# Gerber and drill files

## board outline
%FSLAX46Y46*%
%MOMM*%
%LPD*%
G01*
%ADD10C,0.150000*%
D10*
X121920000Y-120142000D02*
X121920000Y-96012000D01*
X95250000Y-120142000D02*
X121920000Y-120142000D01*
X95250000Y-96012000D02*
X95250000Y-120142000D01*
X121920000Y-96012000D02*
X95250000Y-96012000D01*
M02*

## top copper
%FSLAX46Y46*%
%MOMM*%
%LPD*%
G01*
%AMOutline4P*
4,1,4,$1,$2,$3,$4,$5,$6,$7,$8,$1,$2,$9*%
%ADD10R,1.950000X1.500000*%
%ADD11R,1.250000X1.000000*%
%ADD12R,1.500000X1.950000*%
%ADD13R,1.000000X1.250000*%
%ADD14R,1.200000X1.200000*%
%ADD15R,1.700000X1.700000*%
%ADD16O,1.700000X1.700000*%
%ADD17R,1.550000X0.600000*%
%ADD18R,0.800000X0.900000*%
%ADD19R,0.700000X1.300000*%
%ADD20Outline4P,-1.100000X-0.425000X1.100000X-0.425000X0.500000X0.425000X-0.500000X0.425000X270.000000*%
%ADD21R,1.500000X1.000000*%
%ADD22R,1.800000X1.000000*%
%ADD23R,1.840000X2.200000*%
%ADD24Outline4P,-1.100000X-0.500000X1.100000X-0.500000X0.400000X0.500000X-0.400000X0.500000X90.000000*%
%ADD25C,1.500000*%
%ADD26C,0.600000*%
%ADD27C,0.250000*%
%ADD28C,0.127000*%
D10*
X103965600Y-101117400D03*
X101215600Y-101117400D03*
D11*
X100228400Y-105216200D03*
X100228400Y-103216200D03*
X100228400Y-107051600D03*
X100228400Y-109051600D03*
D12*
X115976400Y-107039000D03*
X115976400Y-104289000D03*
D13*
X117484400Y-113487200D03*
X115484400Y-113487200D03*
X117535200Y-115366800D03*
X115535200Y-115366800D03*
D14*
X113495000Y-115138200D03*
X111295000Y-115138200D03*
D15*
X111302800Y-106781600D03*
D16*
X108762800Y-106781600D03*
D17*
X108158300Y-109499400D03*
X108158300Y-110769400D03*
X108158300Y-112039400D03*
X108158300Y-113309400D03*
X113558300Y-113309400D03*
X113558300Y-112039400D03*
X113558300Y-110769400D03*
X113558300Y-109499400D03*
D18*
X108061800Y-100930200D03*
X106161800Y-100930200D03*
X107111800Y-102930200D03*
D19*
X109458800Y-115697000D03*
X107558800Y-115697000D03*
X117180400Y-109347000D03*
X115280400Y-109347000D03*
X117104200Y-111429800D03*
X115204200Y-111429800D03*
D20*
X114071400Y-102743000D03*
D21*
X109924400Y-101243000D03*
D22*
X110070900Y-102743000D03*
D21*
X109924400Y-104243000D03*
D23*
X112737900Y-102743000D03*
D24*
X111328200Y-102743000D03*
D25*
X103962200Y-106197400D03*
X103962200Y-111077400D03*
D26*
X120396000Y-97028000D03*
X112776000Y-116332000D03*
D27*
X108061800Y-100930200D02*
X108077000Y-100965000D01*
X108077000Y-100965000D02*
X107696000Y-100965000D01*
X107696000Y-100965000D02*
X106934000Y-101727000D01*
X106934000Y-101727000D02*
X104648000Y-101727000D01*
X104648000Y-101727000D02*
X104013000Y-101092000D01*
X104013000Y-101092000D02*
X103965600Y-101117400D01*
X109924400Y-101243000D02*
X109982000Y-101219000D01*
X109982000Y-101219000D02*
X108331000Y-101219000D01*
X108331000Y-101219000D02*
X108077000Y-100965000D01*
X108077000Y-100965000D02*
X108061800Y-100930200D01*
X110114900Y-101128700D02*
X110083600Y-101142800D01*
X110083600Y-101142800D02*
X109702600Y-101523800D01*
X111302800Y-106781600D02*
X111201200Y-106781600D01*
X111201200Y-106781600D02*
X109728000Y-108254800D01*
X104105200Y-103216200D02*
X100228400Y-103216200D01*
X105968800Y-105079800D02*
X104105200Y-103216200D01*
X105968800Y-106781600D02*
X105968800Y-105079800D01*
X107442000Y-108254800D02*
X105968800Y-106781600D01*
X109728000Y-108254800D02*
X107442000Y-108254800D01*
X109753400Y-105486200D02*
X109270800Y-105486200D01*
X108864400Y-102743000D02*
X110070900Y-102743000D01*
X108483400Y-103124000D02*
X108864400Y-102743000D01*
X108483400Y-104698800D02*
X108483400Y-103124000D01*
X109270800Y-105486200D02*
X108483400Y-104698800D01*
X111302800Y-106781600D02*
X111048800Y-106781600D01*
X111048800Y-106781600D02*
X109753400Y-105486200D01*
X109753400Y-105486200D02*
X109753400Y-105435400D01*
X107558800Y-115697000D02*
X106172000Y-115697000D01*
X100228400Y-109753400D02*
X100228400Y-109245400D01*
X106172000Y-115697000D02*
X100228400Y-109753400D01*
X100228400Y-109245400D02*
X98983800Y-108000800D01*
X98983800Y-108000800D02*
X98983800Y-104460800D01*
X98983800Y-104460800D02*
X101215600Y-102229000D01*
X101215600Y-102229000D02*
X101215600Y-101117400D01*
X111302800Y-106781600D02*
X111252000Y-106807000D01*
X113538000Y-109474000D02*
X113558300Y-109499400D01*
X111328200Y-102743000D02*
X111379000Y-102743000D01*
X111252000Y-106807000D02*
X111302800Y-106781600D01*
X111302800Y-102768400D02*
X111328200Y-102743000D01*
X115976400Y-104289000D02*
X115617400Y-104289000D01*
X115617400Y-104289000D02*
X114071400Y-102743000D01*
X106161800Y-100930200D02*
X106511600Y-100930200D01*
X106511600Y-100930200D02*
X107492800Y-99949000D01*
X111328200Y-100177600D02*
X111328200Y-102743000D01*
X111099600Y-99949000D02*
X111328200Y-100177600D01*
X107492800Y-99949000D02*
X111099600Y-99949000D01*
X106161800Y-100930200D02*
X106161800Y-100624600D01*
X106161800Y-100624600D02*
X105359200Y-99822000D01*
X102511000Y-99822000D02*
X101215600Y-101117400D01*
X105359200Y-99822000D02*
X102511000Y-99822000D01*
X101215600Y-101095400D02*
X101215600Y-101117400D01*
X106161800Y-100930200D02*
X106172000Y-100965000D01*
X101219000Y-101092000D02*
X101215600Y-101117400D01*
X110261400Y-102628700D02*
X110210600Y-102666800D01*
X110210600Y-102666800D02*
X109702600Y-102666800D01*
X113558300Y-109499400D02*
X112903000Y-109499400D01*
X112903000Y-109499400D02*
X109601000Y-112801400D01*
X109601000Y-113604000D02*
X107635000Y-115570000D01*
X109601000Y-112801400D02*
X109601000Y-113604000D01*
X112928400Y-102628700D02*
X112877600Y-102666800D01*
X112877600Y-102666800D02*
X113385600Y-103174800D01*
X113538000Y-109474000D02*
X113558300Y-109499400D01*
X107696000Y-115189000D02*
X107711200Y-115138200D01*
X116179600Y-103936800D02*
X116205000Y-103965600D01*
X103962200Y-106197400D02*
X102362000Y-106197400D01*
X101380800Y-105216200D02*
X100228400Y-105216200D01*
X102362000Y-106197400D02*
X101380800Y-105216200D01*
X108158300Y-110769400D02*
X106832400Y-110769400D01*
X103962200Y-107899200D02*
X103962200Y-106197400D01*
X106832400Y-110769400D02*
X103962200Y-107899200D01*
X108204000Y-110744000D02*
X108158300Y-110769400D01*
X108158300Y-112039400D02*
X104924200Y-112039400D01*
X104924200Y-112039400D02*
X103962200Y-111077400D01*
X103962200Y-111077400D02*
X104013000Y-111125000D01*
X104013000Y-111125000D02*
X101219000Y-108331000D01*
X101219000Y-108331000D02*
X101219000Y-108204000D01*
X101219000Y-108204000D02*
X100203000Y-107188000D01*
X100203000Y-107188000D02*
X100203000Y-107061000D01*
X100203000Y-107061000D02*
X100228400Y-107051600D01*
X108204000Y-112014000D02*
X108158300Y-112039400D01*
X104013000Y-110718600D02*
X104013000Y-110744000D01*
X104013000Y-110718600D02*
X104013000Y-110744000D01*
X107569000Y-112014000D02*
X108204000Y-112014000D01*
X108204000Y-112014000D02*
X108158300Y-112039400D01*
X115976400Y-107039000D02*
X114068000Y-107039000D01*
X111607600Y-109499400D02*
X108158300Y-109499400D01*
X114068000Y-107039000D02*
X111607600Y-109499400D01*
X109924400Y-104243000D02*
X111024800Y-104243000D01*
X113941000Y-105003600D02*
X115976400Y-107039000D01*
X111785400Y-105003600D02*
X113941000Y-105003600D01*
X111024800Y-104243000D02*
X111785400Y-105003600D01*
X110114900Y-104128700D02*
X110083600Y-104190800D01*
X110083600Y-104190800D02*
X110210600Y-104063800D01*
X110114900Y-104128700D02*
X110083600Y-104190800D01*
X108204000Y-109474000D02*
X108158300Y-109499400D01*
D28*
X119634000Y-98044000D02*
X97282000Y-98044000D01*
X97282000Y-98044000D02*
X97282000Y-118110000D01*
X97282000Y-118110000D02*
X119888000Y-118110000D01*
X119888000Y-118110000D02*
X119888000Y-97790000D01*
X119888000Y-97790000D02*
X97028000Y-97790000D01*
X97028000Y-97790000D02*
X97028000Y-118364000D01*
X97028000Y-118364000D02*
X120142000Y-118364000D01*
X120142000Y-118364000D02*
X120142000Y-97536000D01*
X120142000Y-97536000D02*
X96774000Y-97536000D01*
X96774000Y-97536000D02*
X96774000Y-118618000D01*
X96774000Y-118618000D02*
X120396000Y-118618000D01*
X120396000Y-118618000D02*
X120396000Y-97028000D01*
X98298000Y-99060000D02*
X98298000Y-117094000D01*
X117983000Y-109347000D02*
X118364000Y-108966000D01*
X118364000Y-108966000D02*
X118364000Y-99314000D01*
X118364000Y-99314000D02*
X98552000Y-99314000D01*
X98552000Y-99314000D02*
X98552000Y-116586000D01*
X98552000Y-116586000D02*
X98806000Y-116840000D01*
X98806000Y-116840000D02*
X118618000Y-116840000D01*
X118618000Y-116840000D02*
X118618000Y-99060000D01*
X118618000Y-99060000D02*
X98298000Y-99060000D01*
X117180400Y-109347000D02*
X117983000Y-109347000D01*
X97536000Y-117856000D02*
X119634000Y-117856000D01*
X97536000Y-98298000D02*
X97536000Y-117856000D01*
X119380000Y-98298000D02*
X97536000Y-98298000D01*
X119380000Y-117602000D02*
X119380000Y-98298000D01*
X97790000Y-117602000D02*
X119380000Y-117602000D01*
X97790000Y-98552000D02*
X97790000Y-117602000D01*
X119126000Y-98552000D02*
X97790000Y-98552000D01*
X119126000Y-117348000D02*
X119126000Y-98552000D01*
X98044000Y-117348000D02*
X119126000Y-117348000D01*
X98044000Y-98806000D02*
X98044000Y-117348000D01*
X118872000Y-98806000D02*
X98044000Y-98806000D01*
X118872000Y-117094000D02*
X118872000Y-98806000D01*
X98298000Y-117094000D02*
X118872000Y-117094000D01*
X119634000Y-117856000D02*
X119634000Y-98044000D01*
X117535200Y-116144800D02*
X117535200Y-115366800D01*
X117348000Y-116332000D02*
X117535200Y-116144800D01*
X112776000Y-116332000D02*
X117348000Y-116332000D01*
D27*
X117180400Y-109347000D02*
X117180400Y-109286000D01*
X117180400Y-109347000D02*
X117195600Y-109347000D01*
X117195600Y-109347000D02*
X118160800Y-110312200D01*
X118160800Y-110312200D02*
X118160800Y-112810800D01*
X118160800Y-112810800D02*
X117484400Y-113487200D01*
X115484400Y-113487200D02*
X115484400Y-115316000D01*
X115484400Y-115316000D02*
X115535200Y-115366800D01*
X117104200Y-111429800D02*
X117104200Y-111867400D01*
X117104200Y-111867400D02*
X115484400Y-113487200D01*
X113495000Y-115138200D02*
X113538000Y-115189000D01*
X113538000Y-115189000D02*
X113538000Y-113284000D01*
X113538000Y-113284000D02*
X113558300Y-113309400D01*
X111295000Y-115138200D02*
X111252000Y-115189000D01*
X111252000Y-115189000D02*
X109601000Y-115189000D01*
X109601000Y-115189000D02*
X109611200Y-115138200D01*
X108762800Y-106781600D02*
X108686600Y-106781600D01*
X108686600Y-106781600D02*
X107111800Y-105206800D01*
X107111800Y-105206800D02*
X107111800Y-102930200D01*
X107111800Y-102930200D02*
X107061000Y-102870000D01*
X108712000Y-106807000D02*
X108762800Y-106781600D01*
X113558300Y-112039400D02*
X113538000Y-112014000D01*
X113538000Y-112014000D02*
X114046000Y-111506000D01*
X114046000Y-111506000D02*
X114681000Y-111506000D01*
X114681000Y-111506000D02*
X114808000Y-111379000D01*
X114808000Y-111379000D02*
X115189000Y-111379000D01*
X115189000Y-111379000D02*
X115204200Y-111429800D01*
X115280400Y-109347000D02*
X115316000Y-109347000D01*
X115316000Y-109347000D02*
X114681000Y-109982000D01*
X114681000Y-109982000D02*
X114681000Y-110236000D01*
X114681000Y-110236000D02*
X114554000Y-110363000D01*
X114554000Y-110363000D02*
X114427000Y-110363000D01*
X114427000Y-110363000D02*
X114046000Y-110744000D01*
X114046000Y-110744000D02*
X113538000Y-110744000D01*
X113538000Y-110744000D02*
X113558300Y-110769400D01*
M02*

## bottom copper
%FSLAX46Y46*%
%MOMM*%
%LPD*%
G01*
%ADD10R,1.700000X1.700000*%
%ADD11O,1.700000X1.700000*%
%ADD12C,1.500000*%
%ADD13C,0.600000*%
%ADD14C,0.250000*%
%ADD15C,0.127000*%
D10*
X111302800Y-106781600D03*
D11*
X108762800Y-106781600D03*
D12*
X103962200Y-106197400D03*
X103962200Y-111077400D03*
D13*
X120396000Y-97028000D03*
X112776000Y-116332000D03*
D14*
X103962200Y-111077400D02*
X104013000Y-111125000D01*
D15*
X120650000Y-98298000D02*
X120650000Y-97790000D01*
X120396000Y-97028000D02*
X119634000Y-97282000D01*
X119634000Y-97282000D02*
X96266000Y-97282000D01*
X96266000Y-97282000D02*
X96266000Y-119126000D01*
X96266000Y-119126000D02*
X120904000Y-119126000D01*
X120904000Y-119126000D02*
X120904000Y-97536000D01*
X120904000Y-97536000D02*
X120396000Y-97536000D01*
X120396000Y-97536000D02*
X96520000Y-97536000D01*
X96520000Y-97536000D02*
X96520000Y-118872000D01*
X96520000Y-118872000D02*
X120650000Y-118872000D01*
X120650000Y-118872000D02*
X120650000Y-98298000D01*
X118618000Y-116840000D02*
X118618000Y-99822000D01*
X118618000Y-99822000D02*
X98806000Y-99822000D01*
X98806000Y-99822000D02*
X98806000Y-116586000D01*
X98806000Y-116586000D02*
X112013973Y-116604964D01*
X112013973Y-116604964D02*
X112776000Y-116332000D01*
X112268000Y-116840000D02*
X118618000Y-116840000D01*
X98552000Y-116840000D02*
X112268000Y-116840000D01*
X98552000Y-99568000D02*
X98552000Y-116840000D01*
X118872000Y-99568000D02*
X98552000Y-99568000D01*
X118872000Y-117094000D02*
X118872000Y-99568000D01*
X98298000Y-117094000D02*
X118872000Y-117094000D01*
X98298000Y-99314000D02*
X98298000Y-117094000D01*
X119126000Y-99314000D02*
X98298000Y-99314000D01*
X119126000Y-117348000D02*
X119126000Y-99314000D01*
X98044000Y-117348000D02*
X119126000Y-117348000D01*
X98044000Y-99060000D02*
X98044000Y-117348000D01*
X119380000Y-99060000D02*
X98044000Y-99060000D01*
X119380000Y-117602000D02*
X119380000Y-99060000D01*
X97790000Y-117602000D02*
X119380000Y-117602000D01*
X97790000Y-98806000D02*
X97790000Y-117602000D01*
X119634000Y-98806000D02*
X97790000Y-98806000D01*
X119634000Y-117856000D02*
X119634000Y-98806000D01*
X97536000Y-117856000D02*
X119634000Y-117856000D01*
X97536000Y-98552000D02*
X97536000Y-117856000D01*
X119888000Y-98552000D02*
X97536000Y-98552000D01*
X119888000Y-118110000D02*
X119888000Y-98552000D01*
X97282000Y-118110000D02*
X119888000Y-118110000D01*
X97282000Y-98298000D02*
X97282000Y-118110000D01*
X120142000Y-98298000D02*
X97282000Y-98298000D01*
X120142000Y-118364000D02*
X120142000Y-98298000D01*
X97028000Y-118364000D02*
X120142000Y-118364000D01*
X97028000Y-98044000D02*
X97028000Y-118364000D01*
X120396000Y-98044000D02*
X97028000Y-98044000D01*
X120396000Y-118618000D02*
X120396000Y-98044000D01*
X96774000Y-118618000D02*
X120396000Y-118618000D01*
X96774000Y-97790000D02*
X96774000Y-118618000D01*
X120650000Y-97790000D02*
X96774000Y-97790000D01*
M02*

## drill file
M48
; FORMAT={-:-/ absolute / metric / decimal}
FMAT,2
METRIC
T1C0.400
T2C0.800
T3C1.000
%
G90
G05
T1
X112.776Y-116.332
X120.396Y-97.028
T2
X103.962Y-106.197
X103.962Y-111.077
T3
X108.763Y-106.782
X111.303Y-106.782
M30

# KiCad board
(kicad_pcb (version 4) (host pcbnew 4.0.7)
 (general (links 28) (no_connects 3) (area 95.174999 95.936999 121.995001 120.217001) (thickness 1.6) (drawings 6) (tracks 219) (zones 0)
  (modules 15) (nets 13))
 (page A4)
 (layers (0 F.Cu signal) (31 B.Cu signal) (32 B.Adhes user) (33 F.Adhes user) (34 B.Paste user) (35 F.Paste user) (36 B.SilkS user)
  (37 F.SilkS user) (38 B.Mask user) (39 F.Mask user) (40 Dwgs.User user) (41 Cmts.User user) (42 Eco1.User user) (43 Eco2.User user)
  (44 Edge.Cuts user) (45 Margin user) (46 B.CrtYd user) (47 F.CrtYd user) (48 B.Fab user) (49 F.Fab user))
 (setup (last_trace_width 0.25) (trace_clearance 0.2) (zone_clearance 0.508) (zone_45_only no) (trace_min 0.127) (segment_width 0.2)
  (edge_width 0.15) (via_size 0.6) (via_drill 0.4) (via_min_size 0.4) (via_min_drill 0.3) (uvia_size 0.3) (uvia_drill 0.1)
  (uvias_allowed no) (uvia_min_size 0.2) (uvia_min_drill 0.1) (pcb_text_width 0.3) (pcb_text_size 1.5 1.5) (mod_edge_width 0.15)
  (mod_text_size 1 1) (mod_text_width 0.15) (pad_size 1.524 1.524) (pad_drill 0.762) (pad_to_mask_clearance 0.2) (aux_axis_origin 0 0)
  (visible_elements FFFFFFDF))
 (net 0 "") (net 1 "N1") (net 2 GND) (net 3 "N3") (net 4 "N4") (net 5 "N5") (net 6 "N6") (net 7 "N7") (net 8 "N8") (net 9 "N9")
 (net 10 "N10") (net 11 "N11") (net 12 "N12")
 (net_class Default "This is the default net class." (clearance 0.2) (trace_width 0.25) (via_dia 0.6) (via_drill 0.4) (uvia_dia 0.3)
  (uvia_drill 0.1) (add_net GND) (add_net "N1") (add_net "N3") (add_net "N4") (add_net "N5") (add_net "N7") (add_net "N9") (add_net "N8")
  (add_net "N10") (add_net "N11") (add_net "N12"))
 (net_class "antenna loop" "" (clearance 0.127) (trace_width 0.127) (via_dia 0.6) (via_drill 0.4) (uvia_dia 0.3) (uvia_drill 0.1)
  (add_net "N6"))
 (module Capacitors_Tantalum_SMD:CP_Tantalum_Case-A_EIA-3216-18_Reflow (layer F.Cu) (at 102.5906 101.1174 180)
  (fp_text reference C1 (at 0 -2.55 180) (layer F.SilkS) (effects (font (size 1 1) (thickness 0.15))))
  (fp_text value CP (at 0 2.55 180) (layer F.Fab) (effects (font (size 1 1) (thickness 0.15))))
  (pad 1 smd rect (at -1.375 0 180) (size 1.95 1.5) (layers F.Cu F.Paste F.Mask) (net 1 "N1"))
  (pad 2 smd rect (at 1.375 0 180) (size 1.95 1.5) (layers F.Cu F.Paste F.Mask) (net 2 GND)))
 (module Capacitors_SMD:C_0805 (layer F.Cu) (at 100.2284 104.2162 90)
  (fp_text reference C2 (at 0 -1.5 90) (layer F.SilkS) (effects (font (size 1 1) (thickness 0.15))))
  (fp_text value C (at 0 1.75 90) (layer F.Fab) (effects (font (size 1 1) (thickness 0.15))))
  (pad 1 smd rect (at -1 0 90) (size 1 1.25) (layers F.Cu F.Paste F.Mask) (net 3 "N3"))
  (pad 2 smd rect (at 1 0 90) (size 1 1.25) (layers F.Cu F.Paste F.Mask) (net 2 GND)))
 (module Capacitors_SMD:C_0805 (layer F.Cu) (at 100.2284 108.0516 270)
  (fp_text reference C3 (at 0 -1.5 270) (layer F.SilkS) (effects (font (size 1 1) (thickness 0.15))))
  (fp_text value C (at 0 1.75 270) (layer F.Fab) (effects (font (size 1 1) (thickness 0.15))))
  (pad 1 smd rect (at -1 0 270) (size 1 1.25) (layers F.Cu F.Paste F.Mask) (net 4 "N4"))
  (pad 2 smd rect (at 1 0 270) (size 1 1.25) (layers F.Cu F.Paste F.Mask) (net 2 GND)))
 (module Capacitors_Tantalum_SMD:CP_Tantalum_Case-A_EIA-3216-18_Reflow (layer F.Cu) (at 115.9764 105.664 90)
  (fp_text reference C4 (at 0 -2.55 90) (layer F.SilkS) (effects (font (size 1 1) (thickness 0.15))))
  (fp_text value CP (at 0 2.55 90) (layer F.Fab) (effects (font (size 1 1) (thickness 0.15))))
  (pad 1 smd rect (at -1.375 0 90) (size 1.95 1.5) (layers F.Cu F.Paste F.Mask) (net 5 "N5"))
  (pad 2 smd rect (at 1.375 0 90) (size 1.95 1.5) (layers F.Cu F.Paste F.Mask) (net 2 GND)))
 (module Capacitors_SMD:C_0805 (layer F.Cu) (at 116.4844 113.4872 180)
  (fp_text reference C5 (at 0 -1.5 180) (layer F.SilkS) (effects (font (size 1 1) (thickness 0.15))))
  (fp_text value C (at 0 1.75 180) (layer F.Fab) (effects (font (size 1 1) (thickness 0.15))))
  (pad 1 smd rect (at -1 0 180) (size 1 1.25) (layers F.Cu F.Paste F.Mask) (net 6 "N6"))
  (pad 2 smd rect (at 1 0 180) (size 1 1.25) (layers F.Cu F.Paste F.Mask) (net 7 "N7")))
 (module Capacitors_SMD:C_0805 (layer F.Cu) (at 116.5352 115.3668 180)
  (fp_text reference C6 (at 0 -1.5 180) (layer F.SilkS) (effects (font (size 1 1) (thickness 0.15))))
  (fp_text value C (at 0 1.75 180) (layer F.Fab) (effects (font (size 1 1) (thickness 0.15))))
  (pad 1 smd rect (at -1 0 180) (size 1 1.25) (layers F.Cu F.Paste F.Mask) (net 6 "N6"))
  (pad 2 smd rect (at 1 0 180) (size 1 1.25) (layers F.Cu F.Paste F.Mask) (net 7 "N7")))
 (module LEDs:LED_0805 (layer F.Cu) (at 112.395 115.1382)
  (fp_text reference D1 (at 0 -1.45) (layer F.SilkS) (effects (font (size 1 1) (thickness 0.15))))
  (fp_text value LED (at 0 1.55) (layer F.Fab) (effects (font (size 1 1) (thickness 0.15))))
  (pad 2 smd rect (at 1.1 0 180) (size 1.2 1.2) (layers F.Cu F.Paste F.Mask) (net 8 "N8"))
  (pad 1 smd rect (at -1.1 0 180) (size 1.2 1.2) (layers F.Cu F.Paste F.Mask) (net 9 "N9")))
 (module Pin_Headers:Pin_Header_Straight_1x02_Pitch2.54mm (layer F.Cu) (at 111.3028 106.7816 270)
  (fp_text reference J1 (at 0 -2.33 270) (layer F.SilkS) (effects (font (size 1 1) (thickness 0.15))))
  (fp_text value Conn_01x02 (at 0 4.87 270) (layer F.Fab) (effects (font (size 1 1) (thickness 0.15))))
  (pad 1 thru_hole rect (at 0 0 270) (size 1.7 1.7) (drill 1) (layers *.Cu *.Mask) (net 2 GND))
  (pad 2 thru_hole oval (at 0 2.54 270) (size 1.7 1.7) (drill 1) (layers *.Cu *.Mask) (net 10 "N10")))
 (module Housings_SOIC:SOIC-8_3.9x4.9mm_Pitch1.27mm (layer F.Cu) (at 110.8583 111.4044)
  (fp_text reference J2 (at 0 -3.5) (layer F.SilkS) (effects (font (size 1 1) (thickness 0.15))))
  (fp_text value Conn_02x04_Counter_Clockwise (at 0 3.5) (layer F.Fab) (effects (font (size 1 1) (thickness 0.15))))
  (pad 1 smd rect (at -2.7 -1.905) (size 1.55 0.6) (layers F.Cu F.Paste F.Mask) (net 5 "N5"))
  (pad 2 smd rect (at -2.7 -0.635) (size 1.55 0.6) (layers F.Cu F.Paste F.Mask) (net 3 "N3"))
  (pad 3 smd rect (at -2.7 0.635) (size 1.55 0.6) (layers F.Cu F.Paste F.Mask) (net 4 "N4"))
  (pad 4 smd rect (at -2.7 1.905) (size 1.55 0.6) (layers F.Cu F.Paste F.Mask))
  (pad 5 smd rect (at 2.7 1.905) (size 1.55 0.6) (layers F.Cu F.Paste F.Mask) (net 8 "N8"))
  (pad 6 smd rect (at 2.7 0.635) (size 1.55 0.6) (layers F.Cu F.Paste F.Mask) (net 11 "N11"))
  (pad 7 smd rect (at 2.7 -0.635) (size 1.55 0.6) (layers F.Cu F.Paste F.Mask) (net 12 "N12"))
  (pad 8 smd rect (at 2.7 -1.905) (size 1.55 0.6) (layers F.Cu F.Paste F.Mask) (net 2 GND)))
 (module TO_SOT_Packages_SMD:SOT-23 (layer F.Cu) (at 107.1118 101.9302 270)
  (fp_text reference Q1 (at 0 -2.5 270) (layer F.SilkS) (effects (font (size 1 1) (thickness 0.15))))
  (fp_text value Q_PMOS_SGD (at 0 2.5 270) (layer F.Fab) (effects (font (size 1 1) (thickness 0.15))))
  (pad 1 smd rect (at -1 -0.95 270) (size 0.9 0.8) (layers F.Cu F.Paste F.Mask) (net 1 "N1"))
  (pad 2 smd rect (at -1 0.95 270) (size 0.9 0.8) (layers F.Cu F.Paste F.Mask) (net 2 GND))
  (pad 3 smd rect (at 1 0 270) (size 0.9 0.8) (layers F.Cu F.Paste F.Mask) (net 10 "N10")))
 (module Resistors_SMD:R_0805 (layer F.Cu) (at 108.5088 115.697 180)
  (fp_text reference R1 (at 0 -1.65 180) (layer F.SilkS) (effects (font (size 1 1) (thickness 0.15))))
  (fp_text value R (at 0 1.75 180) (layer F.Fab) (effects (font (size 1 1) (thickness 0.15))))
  (pad 1 smd rect (at -0.95 0 180) (size 0.7 1.3) (layers F.Cu F.Paste F.Mask) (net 9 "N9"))
  (pad 2 smd rect (at 0.95 0 180) (size 0.7 1.3) (layers F.Cu F.Paste F.Mask) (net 2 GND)))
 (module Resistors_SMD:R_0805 (layer F.Cu) (at 116.2304 109.347 180)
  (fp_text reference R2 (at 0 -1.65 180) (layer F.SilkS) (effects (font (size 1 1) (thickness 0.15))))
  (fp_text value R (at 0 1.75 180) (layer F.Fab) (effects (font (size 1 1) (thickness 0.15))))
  (pad 1 smd rect (at -0.95 0 180) (size 0.7 1.3) (layers F.Cu F.Paste F.Mask) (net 6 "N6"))
  (pad 2 smd rect (at 0.95 0 180) (size 0.7 1.3) (layers F.Cu F.Paste F.Mask) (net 12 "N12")))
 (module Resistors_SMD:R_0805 (layer F.Cu) (at 116.1542 111.4298 180)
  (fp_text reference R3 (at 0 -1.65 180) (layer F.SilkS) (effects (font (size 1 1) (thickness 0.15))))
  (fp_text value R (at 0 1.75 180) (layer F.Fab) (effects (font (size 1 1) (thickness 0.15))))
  (pad 1 smd rect (at -0.95 0 180) (size 0.7 1.3) (layers F.Cu F.Paste F.Mask) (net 7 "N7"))
  (pad 2 smd rect (at 0.95 0 180) (size 0.7 1.3) (layers F.Cu F.Paste F.Mask) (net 11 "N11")))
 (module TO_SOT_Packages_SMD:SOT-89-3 (layer F.Cu) (at 111.4044 102.743)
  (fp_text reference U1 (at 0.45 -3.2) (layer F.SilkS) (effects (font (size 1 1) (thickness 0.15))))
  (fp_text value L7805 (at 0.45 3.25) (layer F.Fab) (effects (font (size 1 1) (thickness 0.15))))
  (pad 2 smd trapezoid (at 2.667 0 270) (size 1.6 0.85) (rect_delta 0 0.6) (layers F.Cu F.Paste F.Mask) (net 2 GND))
  (pad 1 smd rect (at -1.48 -1.5 270) (size 1 1.5) (layers F.Cu F.Paste F.Mask) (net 1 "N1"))
  (pad 2 smd rect (at -1.3335 0 270) (size 1 1.8) (layers F.Cu F.Paste F.Mask) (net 2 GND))
  (pad 3 smd rect (at -1.48 1.5 270) (size 1 1.5) (layers F.Cu F.Paste F.Mask) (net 5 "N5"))
  (pad 2 smd rect (at 1.3335 0 270) (size 2.2 1.84) (layers F.Cu F.Paste F.Mask) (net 2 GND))
  (pad 2 smd trapezoid (at -0.0762 0 90) (size 1.5 1) (rect_delta 0 0.7) (layers F.Cu F.Paste F.Mask) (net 2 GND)))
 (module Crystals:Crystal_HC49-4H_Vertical (layer F.Cu) (at 103.9622 106.1974 270)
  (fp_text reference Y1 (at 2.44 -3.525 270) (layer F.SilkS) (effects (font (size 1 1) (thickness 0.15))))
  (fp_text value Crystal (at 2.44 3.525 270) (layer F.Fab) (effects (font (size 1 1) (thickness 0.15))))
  (pad 1 thru_hole circle (at 0 0 270) (size 1.5 1.5) (drill 0.8) (layers *.Cu *.Mask) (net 3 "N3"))
  (pad 2 thru_hole circle (at 4.88 0 270) (size 1.5 1.5) (drill 0.8) (layers *.Cu *.Mask) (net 4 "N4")))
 (gr_line (start 121.92 120.142) (end 121.92 96.012) (angle 90) (layer Edge.Cuts) (width 0.15))
 (gr_line (start 95.25 120.142) (end 121.92 120.142) (angle 90) (layer Edge.Cuts) (width 0.15))
 (gr_line (start 95.25 96.012) (end 95.25 120.142) (angle 90) (layer Edge.Cuts) (width 0.15))
 (gr_line (start 121.92 96.012) (end 95.25 96.012) (angle 90) (layer Edge.Cuts) (width 0.15))
 (segment (start 108.0618 100.9302) (end 108.077 100.965) (width 0.25) (layer F.Cu) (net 1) (status 80000))
 (segment (start 108.077 100.965) (end 107.696 100.965) (width 0.25) (layer F.Cu) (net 1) (status 80000))
 (segment (start 107.696 100.965) (end 106.934 101.727) (width 0.25) (layer F.Cu) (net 1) (status 80000))
 (segment (start 106.934 101.727) (end 104.648 101.727) (width 0.25) (layer F.Cu) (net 1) (status 80000))
 (segment (start 104.648 101.727) (end 104.013 101.092) (width 0.25) (layer F.Cu) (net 1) (status 80000))
 (segment (start 104.013 101.092) (end 103.9656 101.1174) (width 0.25) (layer F.Cu) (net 1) (status 80000))
 (segment (start 109.9244 101.243) (end 109.982 101.219) (width 0.25) (layer F.Cu) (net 1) (status 80000))
 (segment (start 109.982 101.219) (end 108.331 101.219) (width 0.25) (layer F.Cu) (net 1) (status 80000))
 (segment (start 108.331 101.219) (end 108.077 100.965) (width 0.25) (layer F.Cu) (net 1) (status 80000))
 (segment (start 108.077 100.965) (end 108.0618 100.9302) (width 0.25) (layer F.Cu) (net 1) (status 80000))
 (segment (start 110.1149 101.1287) (end 110.0836 101.1428) (width 0.25) (layer F.Cu) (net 1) (status 80000))
 (segment (start 110.0836 101.1428) (end 109.7026 101.5238) (width 0.25) (layer F.Cu) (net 1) (status 80000))
 (segment (start 111.3028 106.7816) (end 111.2012 106.7816) (width 0.25) (layer F.Cu) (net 2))
 (segment (start 111.2012 106.7816) (end 109.728 108.2548) (width 0.25) (layer F.Cu) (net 2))
 (segment (start 104.1052 103.2162) (end 100.2284 103.2162) (width 0.25) (layer F.Cu) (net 2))
 (segment (start 105.9688 105.0798) (end 104.1052 103.2162) (width 0.25) (layer F.Cu) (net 2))
 (segment (start 105.9688 106.7816) (end 105.9688 105.0798) (width 0.25) (layer F.Cu) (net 2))
 (segment (start 107.442 108.2548) (end 105.9688 106.7816) (width 0.25) (layer F.Cu) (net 2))
 (segment (start 109.728 108.2548) (end 107.442 108.2548) (width 0.25) (layer F.Cu) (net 2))
 (segment (start 109.7534 105.4862) (end 109.2708 105.4862) (width 0.25) (layer F.Cu) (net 2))
 (segment (start 108.8644 102.743) (end 110.0709 102.743) (width 0.25) (layer F.Cu) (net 2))
 (segment (start 108.4834 103.124) (end 108.8644 102.743) (width 0.25) (layer F.Cu) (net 2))
 (segment (start 108.4834 104.6988) (end 108.4834 103.124) (width 0.25) (layer F.Cu) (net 2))
 (segment (start 109.2708 105.4862) (end 108.4834 104.6988) (width 0.25) (layer F.Cu) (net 2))
 (segment (start 111.3028 106.7816) (end 111.0488 106.7816) (width 0.25) (layer F.Cu) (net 2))
 (segment (start 111.0488 106.7816) (end 109.7534 105.4862) (width 0.25) (layer F.Cu) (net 2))
 (segment (start 109.7534 105.4862) (end 109.7534 105.4354) (width 0.25) (layer F.Cu) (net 2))
 (segment (start 107.5588 115.697) (end 106.172 115.697) (width 0.25) (layer F.Cu) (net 2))
 (segment (start 100.2284 109.7534) (end 100.2284 109.2454) (width 0.25) (layer F.Cu) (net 2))
 (segment (start 106.172 115.697) (end 100.2284 109.7534) (width 0.25) (layer F.Cu) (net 2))
 (segment (start 100.2284 109.2454) (end 98.9838 108.0008) (width 0.25) (layer F.Cu) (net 2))
 (segment (start 98.9838 108.0008) (end 98.9838 104.4608) (width 0.25) (layer F.Cu) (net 2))
 (segment (start 98.9838 104.4608) (end 101.2156 102.229) (width 0.25) (layer F.Cu) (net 2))
 (segment (start 101.2156 102.229) (end 101.2156 101.1174) (width 0.25) (layer F.Cu) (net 2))
 (segment (start 111.3028 106.7816) (end 111.252 106.807) (width 0.25) (layer F.Cu) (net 2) (status 80000))
 (segment (start 113.538 109.474) (end 113.5583 109.4994) (width 0.25) (layer F.Cu) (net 2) (status 80000))
 (segment (start 111.3282 102.743) (end 111.379 102.743) (width 0.25) (layer F.Cu) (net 2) (status 80000))
 (segment (start 111.252 106.807) (end 111.3028 106.7816) (width 0.25) (layer F.Cu) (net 2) (status 80000))
 (segment (start 111.3028 102.7684) (end 111.3282 102.743) (width 0.25) (layer F.Cu) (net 2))
 (segment (start 115.9764 104.289) (end 115.6174 104.289) (width 0.25) (layer F.Cu) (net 2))
 (segment (start 115.6174 104.289) (end 114.0714 102.743) (width 0.25) (layer F.Cu) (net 2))
 (segment (start 106.1618 100.9302) (end 106.5116 100.9302) (width 0.25) (layer F.Cu) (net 2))
 (segment (start 106.5116 100.9302) (end 107.4928 99.949) (width 0.25) (layer F.Cu) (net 2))
 (segment (start 111.3282 100.1776) (end 111.3282 102.743) (width 0.25) (layer F.Cu) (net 2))
 (segment (start 111.0996 99.949) (end 111.3282 100.1776) (width 0.25) (layer F.Cu) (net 2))
 (segment (start 107.4928 99.949) (end 111.0996 99.949) (width 0.25) (layer F.Cu) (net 2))
 (segment (start 106.1618 100.9302) (end 106.1618 100.6246) (width 0.25) (layer F.Cu) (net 2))
 (segment (start 106.1618 100.6246) (end 105.3592 99.822) (width 0.25) (layer F.Cu) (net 2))
 (segment (start 102.511 99.822) (end 101.2156 101.1174) (width 0.25) (layer F.Cu) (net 2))
 (segment (start 105.3592 99.822) (end 102.511 99.822) (width 0.25) (layer F.Cu) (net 2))
 (segment (start 101.2156 101.0954) (end 101.2156 101.1174) (width 0.25) (layer F.Cu) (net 2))
 (segment (start 106.1618 100.9302) (end 106.172 100.965) (width 0.25) (layer F.Cu) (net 2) (status 80000))
 (segment (start 101.219 101.092) (end 101.2156 101.1174) (width 0.25) (layer F.Cu) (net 2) (status 80000))
 (segment (start 110.2614 102.6287) (end 110.2106 102.6668) (width 0.25) (layer F.Cu) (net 2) (status 80000))
 (segment (start 110.2106 102.6668) (end 109.7026 102.6668) (width 0.25) (layer F.Cu) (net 2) (status 80000))
 (segment (start 113.5583 109.4994) (end 112.903 109.4994) (width 0.25) (layer F.Cu) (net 2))
 (segment (start 112.903 109.4994) (end 109.601 112.8014) (width 0.25) (layer F.Cu) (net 2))
 (segment (start 109.601 113.604) (end 107.635 115.57) (width 0.25) (layer F.Cu) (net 2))
 (segment (start 109.601 112.8014) (end 109.601 113.604) (width 0.25) (layer F.Cu) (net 2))
 (segment (start 112.9284 102.6287) (end 112.8776 102.6668) (width 0.25) (layer F.Cu) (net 2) (status 80000))
 (segment (start 112.8776 102.6668) (end 113.3856 103.1748) (width 0.25) (layer F.Cu) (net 2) (status 80000))
 (segment (start 113.538 109.474) (end 113.5583 109.4994) (width 0.25) (layer F.Cu) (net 2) (status 80000))
 (segment (start 107.696 115.189) (end 107.7112 115.1382) (width 0.25) (layer F.Cu) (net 2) (status 80000))
 (segment (start 116.1796 103.9368) (end 116.205 103.9656) (width 0.25) (layer F.Cu) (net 2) (status 80000))
 (segment (start 103.9622 106.1974) (end 102.362 106.1974) (width 0.25) (layer F.Cu) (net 3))
 (segment (start 101.3808 105.2162) (end 100.2284 105.2162) (width 0.25) (layer F.Cu) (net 3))
 (segment (start 102.362 106.1974) (end 101.3808 105.2162) (width 0.25) (layer F.Cu) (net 3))
 (segment (start 108.1583 110.7694) (end 106.8324 110.7694) (width 0.25) (layer F.Cu) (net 3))
 (segment (start 103.9622 107.8992) (end 103.9622 106.1974) (width 0.25) (layer F.Cu) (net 3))
 (segment (start 106.8324 110.7694) (end 103.9622 107.8992) (width 0.25) (layer F.Cu) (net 3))
 (segment (start 108.204 110.744) (end 108.1583 110.7694) (width 0.25) (layer F.Cu) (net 3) (status 80000))
 (segment (start 108.1583 112.0394) (end 104.9242 112.0394) (width 0.25) (layer F.Cu) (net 4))
 (segment (start 104.9242 112.0394) (end 103.9622 111.0774) (width 0.25) (layer F.Cu) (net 4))
 (segment (start 103.9622 111.0774) (end 104.013 111.125) (width 0.25) (layer F.Cu) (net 4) (status 80000))
 (segment (start 104.013 111.125) (end 101.219 108.331) (width 0.25) (layer F.Cu) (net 4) (status 80000))
 (segment (start 101.219 108.331) (end 101.219 108.204) (width 0.25) (layer F.Cu) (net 4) (status 80000))
 (segment (start 101.219 108.204) (end 100.203 107.188) (width 0.25) (layer F.Cu) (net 4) (status 80000))
 (segment (start 100.203 107.188) (end 100.203 107.061) (width 0.25) (layer F.Cu) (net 4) (status 80000))
 (segment (start 100.203 107.061) (end 100.2284 107.0516) (width 0.25) (layer F.Cu) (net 4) (status 80000))
 (segment (start 103.9622 111.0774) (end 104.013 111.125) (width 0.25) (layer B.Cu) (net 4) (status 80000))
 (segment (start 108.204 112.014) (end 108.1583 112.0394) (width 0.25) (layer F.Cu) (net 4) (status 80000))
 (segment (start 104.013 110.7186) (end 104.013 110.744) (width 0.25) (layer F.Cu) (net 4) (status 80000))
 (segment (start 104.013 110.7186) (end 104.013 110.744) (width 0.25) (layer F.Cu) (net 4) (status 80000))
 (segment (start 107.569 112.014) (end 108.204 112.014) (width 0.25) (layer F.Cu) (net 4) (status 80000))
 (segment (start 108.204 112.014) (end 108.1583 112.0394) (width 0.25) (layer F.Cu) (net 4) (status 80000))
 (segment (start 115.9764 107.039) (end 114.068 107.039) (width 0.25) (layer F.Cu) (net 5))
 (segment (start 111.6076 109.4994) (end 108.1583 109.4994) (width 0.25) (layer F.Cu) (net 5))
 (segment (start 114.068 107.039) (end 111.6076 109.4994) (width 0.25) (layer F.Cu) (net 5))
 (segment (start 109.9244 104.243) (end 111.0248 104.243) (width 0.25) (layer F.Cu) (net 5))
 (segment (start 113.941 105.0036) (end 115.9764 107.039) (width 0.25) (layer F.Cu) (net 5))
 (segment (start 111.7854 105.0036) (end 113.941 105.0036) (width 0.25) (layer F.Cu) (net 5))
 (segment (start 111.0248 104.243) (end 111.7854 105.0036) (width 0.25) (layer F.Cu) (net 5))
 (segment (start 110.1149 104.1287) (end 110.0836 104.1908) (width 0.25) (layer F.Cu) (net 5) (status 80000))
 (segment (start 110.0836 104.1908) (end 110.2106 104.0638) (width 0.25) (layer F.Cu) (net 5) (status 80000))
 (segment (start 110.1149 104.1287) (end 110.0836 104.1908) (width 0.25) (layer F.Cu) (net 5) (status 80000))
 (segment (start 108.204 109.474) (end 108.1583 109.4994) (width 0.25) (layer F.Cu) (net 5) (status 80000))
 (segment (start 120.65 98.298) (end 120.65 97.79) (width 0.127) (layer B.Cu) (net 6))
 (segment (start 119.634 98.044) (end 97.282 98.044) (width 0.127) (layer F.Cu) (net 6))
 (segment (start 97.282 98.044) (end 97.282 118.11) (width 0.127) (layer F.Cu) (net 6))
 (segment (start 97.282 118.11) (end 119.888 118.11) (width 0.127) (layer F.Cu) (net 6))
 (segment (start 119.888 118.11) (end 119.888 97.79) (width 0.127) (layer F.Cu) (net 6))
 (segment (start 119.888 97.79) (end 97.028 97.79) (width 0.127) (layer F.Cu) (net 6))
 (segment (start 97.028 97.79) (end 97.028 118.364) (width 0.127) (layer F.Cu) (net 6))
 (segment (start 97.028 118.364) (end 120.142 118.364) (width 0.127) (layer F.Cu) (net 6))
 (segment (start 120.142 118.364) (end 120.142 97.536) (width 0.127) (layer F.Cu) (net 6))
 (segment (start 120.142 97.536) (end 96.774 97.536) (width 0.127) (layer F.Cu) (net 6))
 (segment (start 96.774 97.536) (end 96.774 118.618) (width 0.127) (layer F.Cu) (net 6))
 (segment (start 96.774 118.618) (end 120.396 118.618) (width 0.127) (layer F.Cu) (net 6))
 (segment (start 120.396 118.618) (end 120.396 97.028) (width 0.127) (layer F.Cu) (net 6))
 (via (at 120.396 97.028) (size 0.6) (drill 0.4) (layers F.Cu B.Cu) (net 6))
 (segment (start 120.396 97.028) (end 119.634 97.282) (width 0.127) (layer B.Cu) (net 6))
 (segment (start 119.634 97.282) (end 96.266 97.282) (width 0.127) (layer B.Cu) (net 6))
 (segment (start 96.266 97.282) (end 96.266 119.126) (width 0.127) (layer B.Cu) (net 6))
 (segment (start 96.266 119.126) (end 120.904 119.126) (width 0.127) (layer B.Cu) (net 6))
 (segment (start 120.904 119.126) (end 120.904 97.536) (width 0.127) (layer B.Cu) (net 6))
 (segment (start 120.904 97.536) (end 120.396 97.536) (width 0.127) (layer B.Cu) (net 6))
 (segment (start 120.396 97.536) (end 96.52 97.536) (width 0.127) (layer B.Cu) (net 6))
 (segment (start 96.52 97.536) (end 96.52 118.872) (width 0.127) (layer B.Cu) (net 6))
 (segment (start 96.52 118.872) (end 120.65 118.872) (width 0.127) (layer B.Cu) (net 6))
 (segment (start 120.65 118.872) (end 120.65 98.298) (width 0.127) (layer B.Cu) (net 6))
 (segment (start 98.298 99.06) (end 98.298 117.094) (width 0.127) (layer F.Cu) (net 6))
 (segment (start 117.983 109.347) (end 118.364 108.966) (width 0.127) (layer F.Cu) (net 6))
 (segment (start 118.364 108.966) (end 118.364 99.314) (width 0.127) (layer F.Cu) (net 6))
 (segment (start 118.364 99.314) (end 98.552 99.314) (width 0.127) (layer F.Cu) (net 6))
 (segment (start 98.552 99.314) (end 98.552 116.586) (width 0.127) (layer F.Cu) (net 6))
 (segment (start 98.552 116.586) (end 98.806 116.84) (width 0.127) (layer F.Cu) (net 6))
 (segment (start 98.806 116.84) (end 118.618 116.84) (width 0.127) (layer F.Cu) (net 6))
 (segment (start 118.618 116.84) (end 118.618 99.06) (width 0.127) (layer F.Cu) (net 6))
 (segment (start 118.618 99.06) (end 98.298 99.06) (width 0.127) (layer F.Cu) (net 6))
 (segment (start 117.1804 109.347) (end 117.983 109.347) (width 0.127) (layer F.Cu) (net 6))
 (segment (start 97.536 117.856) (end 119.634 117.856) (width 0.127) (layer F.Cu) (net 6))
 (segment (start 97.536 98.298) (end 97.536 117.856) (width 0.127) (layer F.Cu) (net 6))
 (segment (start 119.38 98.298) (end 97.536 98.298) (width 0.127) (layer F.Cu) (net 6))
 (segment (start 119.38 117.602) (end 119.38 98.298) (width 0.127) (layer F.Cu) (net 6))
 (segment (start 97.79 117.602) (end 119.38 117.602) (width 0.127) (layer F.Cu) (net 6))
 (segment (start 97.79 98.552) (end 97.79 117.602) (width 0.127) (layer F.Cu) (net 6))
 (segment (start 119.126 98.552) (end 97.79 98.552) (width 0.127) (layer F.Cu) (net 6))
 (segment (start 119.126 117.348) (end 119.126 98.552) (width 0.127) (layer F.Cu) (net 6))
 (segment (start 98.044 117.348) (end 119.126 117.348) (width 0.127) (layer F.Cu) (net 6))
 (segment (start 98.044 98.806) (end 98.044 117.348) (width 0.127) (layer F.Cu) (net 6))
 (segment (start 118.872 98.806) (end 98.044 98.806) (width 0.127) (layer F.Cu) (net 6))
 (segment (start 118.872 117.094) (end 118.872 98.806) (width 0.127) (layer F.Cu) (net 6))
 (segment (start 98.298 117.094) (end 118.872 117.094) (width 0.127) (layer F.Cu) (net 6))
 (segment (start 119.634 117.856) (end 119.634 98.044) (width 0.127) (layer F.Cu) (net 6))
 (segment (start 117.5352 116.1448) (end 117.5352 115.3668) (width 0.127) (layer F.Cu) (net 6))
 (segment (start 117.348 116.332) (end 117.5352 116.1448) (width 0.127) (layer F.Cu) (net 6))
 (segment (start 112.776 116.332) (end 117.348 116.332) (width 0.127) (layer F.Cu) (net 6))
 (via (at 112.776 116.332) (size 0.6) (drill 0.4) (layers F.Cu B.Cu) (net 6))
 (segment (start 118.618 116.84) (end 118.618 99.822) (width 0.127) (layer B.Cu) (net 6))
 (segment (start 118.618 99.822) (end 98.806 99.822) (width 0.127) (layer B.Cu) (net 6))
 (segment (start 98.806 99.822) (end 98.806 116.586) (width 0.127) (layer B.Cu) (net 6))
 (segment (start 98.806 116.586) (end 112.013973 116.604964) (width 0.127) (layer B.Cu) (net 6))
 (segment (start 112.013973 116.604964) (end 112.776 116.332) (width 0.127) (layer B.Cu) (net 6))
 (segment (start 112.268 116.84) (end 118.618 116.84) (width 0.127) (layer B.Cu) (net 6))
 (segment (start 98.552 116.84) (end 112.268 116.84) (width 0.127) (layer B.Cu) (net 6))
 (segment (start 98.552 99.568) (end 98.552 116.84) (width 0.127) (layer B.Cu) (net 6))
 (segment (start 118.872 99.568) (end 98.552 99.568) (width 0.127) (layer B.Cu) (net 6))
 (segment (start 118.872 117.094) (end 118.872 99.568) (width 0.127) (layer B.Cu) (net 6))
 (segment (start 98.298 117.094) (end 118.872 117.094) (width 0.127) (layer B.Cu) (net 6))
 (segment (start 98.298 99.314) (end 98.298 117.094) (width 0.127) (layer B.Cu) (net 6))
 (segment (start 119.126 99.314) (end 98.298 99.314) (width 0.127) (layer B.Cu) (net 6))
 (segment (start 119.126 117.348) (end 119.126 99.314) (width 0.127) (layer B.Cu) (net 6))
 (segment (start 98.044 117.348) (end 119.126 117.348) (width 0.127) (layer B.Cu) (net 6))
 (segment (start 98.044 99.06) (end 98.044 117.348) (width 0.127) (layer B.Cu) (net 6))
 (segment (start 119.38 99.06) (end 98.044 99.06) (width 0.127) (layer B.Cu) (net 6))
 (segment (start 119.38 117.602) (end 119.38 99.06) (width 0.127) (layer B.Cu) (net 6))
 (segment (start 97.79 117.602) (end 119.38 117.602) (width 0.127) (layer B.Cu) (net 6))
 (segment (start 97.79 98.806) (end 97.79 117.602) (width 0.127) (layer B.Cu) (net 6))
 (segment (start 119.634 98.806) (end 97.79 98.806) (width 0.127) (layer B.Cu) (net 6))
 (segment (start 119.634 117.856) (end 119.634 98.806) (width 0.127) (layer B.Cu) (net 6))
 (segment (start 97.536 117.856) (end 119.634 117.856) (width 0.127) (layer B.Cu) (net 6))
 (segment (start 97.536 98.552) (end 97.536 117.856) (width 0.127) (layer B.Cu) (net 6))
 (segment (start 119.888 98.552) (end 97.536 98.552) (width 0.127) (layer B.Cu) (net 6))
 (segment (start 119.888 118.11) (end 119.888 98.552) (width 0.127) (layer B.Cu) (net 6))
 (segment (start 97.282 118.11) (end 119.888 118.11) (width 0.127) (layer B.Cu) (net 6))
 (segment (start 97.282 98.298) (end 97.282 118.11) (width 0.127) (layer B.Cu) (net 6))
 (segment (start 120.142 98.298) (end 97.282 98.298) (width 0.127) (layer B.Cu) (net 6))
 (segment (start 120.142 118.364) (end 120.142 98.298) (width 0.127) (layer B.Cu) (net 6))
 (segment (start 97.028 118.364) (end 120.142 118.364) (width 0.127) (layer B.Cu) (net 6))
 (segment (start 97.028 98.044) (end 97.028 118.364) (width 0.127) (layer B.Cu) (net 6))
 (segment (start 120.396 98.044) (end 97.028 98.044) (width 0.127) (layer B.Cu) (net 6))
 (segment (start 120.396 118.618) (end 120.396 98.044) (width 0.127) (layer B.Cu) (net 6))
 (segment (start 96.774 118.618) (end 120.396 118.618) (width 0.127) (layer B.Cu) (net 6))
 (segment (start 96.774 97.79) (end 96.774 118.618) (width 0.127) (layer B.Cu) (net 6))
 (segment (start 120.65 97.79) (end 96.774 97.79) (width 0.127) (layer B.Cu) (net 6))
 (segment (start 117.1804 109.347) (end 117.1804 109.286) (width 0.25) (layer F.Cu) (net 6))
 (segment (start 117.1804 109.347) (end 117.1956 109.347) (width 0.25) (layer F.Cu) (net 6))
 (segment (start 117.1956 109.347) (end 118.1608 110.3122) (width 0.25) (layer F.Cu) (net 6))
 (segment (start 118.1608 110.3122) (end 118.1608 112.8108) (width 0.25) (layer F.Cu) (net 6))
 (segment (start 118.1608 112.8108) (end 117.4844 113.4872) (width 0.25) (layer F.Cu) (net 6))
 (segment (start 115.4844 113.4872) (end 115.4844 115.316) (width 0.25) (layer F.Cu) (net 7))
 (segment (start 115.4844 115.316) (end 115.5352 115.3668) (width 0.25) (layer F.Cu) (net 7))
 (segment (start 117.1042 111.4298) (end 117.1042 111.8674) (width 0.25) (layer F.Cu) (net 7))
 (segment (start 117.1042 111.8674) (end 115.4844 113.4872) (width 0.25) (layer F.Cu) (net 7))
 (segment (start 113.495 115.1382) (end 113.538 115.189) (width 0.25) (layer F.Cu) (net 8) (status 80000))
 (segment (start 113.538 115.189) (end 113.538 113.284) (width 0.25) (layer F.Cu) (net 8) (status 80000))
 (segment (start 113.538 113.284) (end 113.5583 113.3094) (width 0.25) (layer F.Cu) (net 8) (status 80000))
 (segment (start 111.295 115.1382) (end 111.252 115.189) (width 0.25) (layer F.Cu) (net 9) (status 80000))
 (segment (start 111.252 115.189) (end 109.601 115.189) (width 0.25) (layer F.Cu) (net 9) (status 80000))
 (segment (start 109.601 115.189) (end 109.6112 115.1382) (width 0.25) (layer F.Cu) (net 9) (status 80000))
 (segment (start 108.7628 106.7816) (end 108.6866 106.7816) (width 0.25) (layer F.Cu) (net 10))
 (segment (start 108.6866 106.7816) (end 107.1118 105.2068) (width 0.25) (layer F.Cu) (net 10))
 (segment (start 107.1118 105.2068) (end 107.1118 102.9302) (width 0.25) (layer F.Cu) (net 10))
 (segment (start 107.1118 102.9302) (end 107.061 102.87) (width 0.25) (layer F.Cu) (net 10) (status 80000))
 (segment (start 108.712 106.807) (end 108.7628 106.7816) (width 0.25) (layer F.Cu) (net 10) (status 80000))
 (segment (start 113.5583 112.0394) (end 113.538 112.014) (width 0.25) (layer F.Cu) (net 11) (status 80000))
 (segment (start 113.538 112.014) (end 114.046 111.506) (width 0.25) (layer F.Cu) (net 11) (status 80000))
 (segment (start 114.046 111.506) (end 114.681 111.506) (width 0.25) (layer F.Cu) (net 11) (status 80000))
 (segment (start 114.681 111.506) (end 114.808 111.379) (width 0.25) (layer F.Cu) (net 11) (status 80000))
 (segment (start 114.808 111.379) (end 115.189 111.379) (width 0.25) (layer F.Cu) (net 11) (status 80000))
 (segment (start 115.189 111.379) (end 115.2042 111.4298) (width 0.25) (layer F.Cu) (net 11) (status 80000))
 (segment (start 115.2804 109.347) (end 115.316 109.347) (width 0.25) (layer F.Cu) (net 12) (status 80000))
 (segment (start 115.316 109.347) (end 114.681 109.982) (width 0.25) (layer F.Cu) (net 12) (status 80000))
 (segment (start 114.681 109.982) (end 114.681 110.236) (width 0.25) (layer F.Cu) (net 12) (status 80000))
 (segment (start 114.681 110.236) (end 114.554 110.363) (width 0.25) (layer F.Cu) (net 12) (status 80000))
 (segment (start 114.554 110.363) (end 114.427 110.363) (width 0.25) (layer F.Cu) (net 12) (status 80000))
 (segment (start 114.427 110.363) (end 114.046 110.744) (width 0.25) (layer F.Cu) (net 12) (status 80000))
 (segment (start 114.046 110.744) (end 113.538 110.744) (width 0.25) (layer F.Cu) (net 12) (status 80000))
 (segment (start 113.538 110.744) (end 113.5583 110.7694) (width 0.25) (layer F.Cu) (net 12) (status 80000)))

